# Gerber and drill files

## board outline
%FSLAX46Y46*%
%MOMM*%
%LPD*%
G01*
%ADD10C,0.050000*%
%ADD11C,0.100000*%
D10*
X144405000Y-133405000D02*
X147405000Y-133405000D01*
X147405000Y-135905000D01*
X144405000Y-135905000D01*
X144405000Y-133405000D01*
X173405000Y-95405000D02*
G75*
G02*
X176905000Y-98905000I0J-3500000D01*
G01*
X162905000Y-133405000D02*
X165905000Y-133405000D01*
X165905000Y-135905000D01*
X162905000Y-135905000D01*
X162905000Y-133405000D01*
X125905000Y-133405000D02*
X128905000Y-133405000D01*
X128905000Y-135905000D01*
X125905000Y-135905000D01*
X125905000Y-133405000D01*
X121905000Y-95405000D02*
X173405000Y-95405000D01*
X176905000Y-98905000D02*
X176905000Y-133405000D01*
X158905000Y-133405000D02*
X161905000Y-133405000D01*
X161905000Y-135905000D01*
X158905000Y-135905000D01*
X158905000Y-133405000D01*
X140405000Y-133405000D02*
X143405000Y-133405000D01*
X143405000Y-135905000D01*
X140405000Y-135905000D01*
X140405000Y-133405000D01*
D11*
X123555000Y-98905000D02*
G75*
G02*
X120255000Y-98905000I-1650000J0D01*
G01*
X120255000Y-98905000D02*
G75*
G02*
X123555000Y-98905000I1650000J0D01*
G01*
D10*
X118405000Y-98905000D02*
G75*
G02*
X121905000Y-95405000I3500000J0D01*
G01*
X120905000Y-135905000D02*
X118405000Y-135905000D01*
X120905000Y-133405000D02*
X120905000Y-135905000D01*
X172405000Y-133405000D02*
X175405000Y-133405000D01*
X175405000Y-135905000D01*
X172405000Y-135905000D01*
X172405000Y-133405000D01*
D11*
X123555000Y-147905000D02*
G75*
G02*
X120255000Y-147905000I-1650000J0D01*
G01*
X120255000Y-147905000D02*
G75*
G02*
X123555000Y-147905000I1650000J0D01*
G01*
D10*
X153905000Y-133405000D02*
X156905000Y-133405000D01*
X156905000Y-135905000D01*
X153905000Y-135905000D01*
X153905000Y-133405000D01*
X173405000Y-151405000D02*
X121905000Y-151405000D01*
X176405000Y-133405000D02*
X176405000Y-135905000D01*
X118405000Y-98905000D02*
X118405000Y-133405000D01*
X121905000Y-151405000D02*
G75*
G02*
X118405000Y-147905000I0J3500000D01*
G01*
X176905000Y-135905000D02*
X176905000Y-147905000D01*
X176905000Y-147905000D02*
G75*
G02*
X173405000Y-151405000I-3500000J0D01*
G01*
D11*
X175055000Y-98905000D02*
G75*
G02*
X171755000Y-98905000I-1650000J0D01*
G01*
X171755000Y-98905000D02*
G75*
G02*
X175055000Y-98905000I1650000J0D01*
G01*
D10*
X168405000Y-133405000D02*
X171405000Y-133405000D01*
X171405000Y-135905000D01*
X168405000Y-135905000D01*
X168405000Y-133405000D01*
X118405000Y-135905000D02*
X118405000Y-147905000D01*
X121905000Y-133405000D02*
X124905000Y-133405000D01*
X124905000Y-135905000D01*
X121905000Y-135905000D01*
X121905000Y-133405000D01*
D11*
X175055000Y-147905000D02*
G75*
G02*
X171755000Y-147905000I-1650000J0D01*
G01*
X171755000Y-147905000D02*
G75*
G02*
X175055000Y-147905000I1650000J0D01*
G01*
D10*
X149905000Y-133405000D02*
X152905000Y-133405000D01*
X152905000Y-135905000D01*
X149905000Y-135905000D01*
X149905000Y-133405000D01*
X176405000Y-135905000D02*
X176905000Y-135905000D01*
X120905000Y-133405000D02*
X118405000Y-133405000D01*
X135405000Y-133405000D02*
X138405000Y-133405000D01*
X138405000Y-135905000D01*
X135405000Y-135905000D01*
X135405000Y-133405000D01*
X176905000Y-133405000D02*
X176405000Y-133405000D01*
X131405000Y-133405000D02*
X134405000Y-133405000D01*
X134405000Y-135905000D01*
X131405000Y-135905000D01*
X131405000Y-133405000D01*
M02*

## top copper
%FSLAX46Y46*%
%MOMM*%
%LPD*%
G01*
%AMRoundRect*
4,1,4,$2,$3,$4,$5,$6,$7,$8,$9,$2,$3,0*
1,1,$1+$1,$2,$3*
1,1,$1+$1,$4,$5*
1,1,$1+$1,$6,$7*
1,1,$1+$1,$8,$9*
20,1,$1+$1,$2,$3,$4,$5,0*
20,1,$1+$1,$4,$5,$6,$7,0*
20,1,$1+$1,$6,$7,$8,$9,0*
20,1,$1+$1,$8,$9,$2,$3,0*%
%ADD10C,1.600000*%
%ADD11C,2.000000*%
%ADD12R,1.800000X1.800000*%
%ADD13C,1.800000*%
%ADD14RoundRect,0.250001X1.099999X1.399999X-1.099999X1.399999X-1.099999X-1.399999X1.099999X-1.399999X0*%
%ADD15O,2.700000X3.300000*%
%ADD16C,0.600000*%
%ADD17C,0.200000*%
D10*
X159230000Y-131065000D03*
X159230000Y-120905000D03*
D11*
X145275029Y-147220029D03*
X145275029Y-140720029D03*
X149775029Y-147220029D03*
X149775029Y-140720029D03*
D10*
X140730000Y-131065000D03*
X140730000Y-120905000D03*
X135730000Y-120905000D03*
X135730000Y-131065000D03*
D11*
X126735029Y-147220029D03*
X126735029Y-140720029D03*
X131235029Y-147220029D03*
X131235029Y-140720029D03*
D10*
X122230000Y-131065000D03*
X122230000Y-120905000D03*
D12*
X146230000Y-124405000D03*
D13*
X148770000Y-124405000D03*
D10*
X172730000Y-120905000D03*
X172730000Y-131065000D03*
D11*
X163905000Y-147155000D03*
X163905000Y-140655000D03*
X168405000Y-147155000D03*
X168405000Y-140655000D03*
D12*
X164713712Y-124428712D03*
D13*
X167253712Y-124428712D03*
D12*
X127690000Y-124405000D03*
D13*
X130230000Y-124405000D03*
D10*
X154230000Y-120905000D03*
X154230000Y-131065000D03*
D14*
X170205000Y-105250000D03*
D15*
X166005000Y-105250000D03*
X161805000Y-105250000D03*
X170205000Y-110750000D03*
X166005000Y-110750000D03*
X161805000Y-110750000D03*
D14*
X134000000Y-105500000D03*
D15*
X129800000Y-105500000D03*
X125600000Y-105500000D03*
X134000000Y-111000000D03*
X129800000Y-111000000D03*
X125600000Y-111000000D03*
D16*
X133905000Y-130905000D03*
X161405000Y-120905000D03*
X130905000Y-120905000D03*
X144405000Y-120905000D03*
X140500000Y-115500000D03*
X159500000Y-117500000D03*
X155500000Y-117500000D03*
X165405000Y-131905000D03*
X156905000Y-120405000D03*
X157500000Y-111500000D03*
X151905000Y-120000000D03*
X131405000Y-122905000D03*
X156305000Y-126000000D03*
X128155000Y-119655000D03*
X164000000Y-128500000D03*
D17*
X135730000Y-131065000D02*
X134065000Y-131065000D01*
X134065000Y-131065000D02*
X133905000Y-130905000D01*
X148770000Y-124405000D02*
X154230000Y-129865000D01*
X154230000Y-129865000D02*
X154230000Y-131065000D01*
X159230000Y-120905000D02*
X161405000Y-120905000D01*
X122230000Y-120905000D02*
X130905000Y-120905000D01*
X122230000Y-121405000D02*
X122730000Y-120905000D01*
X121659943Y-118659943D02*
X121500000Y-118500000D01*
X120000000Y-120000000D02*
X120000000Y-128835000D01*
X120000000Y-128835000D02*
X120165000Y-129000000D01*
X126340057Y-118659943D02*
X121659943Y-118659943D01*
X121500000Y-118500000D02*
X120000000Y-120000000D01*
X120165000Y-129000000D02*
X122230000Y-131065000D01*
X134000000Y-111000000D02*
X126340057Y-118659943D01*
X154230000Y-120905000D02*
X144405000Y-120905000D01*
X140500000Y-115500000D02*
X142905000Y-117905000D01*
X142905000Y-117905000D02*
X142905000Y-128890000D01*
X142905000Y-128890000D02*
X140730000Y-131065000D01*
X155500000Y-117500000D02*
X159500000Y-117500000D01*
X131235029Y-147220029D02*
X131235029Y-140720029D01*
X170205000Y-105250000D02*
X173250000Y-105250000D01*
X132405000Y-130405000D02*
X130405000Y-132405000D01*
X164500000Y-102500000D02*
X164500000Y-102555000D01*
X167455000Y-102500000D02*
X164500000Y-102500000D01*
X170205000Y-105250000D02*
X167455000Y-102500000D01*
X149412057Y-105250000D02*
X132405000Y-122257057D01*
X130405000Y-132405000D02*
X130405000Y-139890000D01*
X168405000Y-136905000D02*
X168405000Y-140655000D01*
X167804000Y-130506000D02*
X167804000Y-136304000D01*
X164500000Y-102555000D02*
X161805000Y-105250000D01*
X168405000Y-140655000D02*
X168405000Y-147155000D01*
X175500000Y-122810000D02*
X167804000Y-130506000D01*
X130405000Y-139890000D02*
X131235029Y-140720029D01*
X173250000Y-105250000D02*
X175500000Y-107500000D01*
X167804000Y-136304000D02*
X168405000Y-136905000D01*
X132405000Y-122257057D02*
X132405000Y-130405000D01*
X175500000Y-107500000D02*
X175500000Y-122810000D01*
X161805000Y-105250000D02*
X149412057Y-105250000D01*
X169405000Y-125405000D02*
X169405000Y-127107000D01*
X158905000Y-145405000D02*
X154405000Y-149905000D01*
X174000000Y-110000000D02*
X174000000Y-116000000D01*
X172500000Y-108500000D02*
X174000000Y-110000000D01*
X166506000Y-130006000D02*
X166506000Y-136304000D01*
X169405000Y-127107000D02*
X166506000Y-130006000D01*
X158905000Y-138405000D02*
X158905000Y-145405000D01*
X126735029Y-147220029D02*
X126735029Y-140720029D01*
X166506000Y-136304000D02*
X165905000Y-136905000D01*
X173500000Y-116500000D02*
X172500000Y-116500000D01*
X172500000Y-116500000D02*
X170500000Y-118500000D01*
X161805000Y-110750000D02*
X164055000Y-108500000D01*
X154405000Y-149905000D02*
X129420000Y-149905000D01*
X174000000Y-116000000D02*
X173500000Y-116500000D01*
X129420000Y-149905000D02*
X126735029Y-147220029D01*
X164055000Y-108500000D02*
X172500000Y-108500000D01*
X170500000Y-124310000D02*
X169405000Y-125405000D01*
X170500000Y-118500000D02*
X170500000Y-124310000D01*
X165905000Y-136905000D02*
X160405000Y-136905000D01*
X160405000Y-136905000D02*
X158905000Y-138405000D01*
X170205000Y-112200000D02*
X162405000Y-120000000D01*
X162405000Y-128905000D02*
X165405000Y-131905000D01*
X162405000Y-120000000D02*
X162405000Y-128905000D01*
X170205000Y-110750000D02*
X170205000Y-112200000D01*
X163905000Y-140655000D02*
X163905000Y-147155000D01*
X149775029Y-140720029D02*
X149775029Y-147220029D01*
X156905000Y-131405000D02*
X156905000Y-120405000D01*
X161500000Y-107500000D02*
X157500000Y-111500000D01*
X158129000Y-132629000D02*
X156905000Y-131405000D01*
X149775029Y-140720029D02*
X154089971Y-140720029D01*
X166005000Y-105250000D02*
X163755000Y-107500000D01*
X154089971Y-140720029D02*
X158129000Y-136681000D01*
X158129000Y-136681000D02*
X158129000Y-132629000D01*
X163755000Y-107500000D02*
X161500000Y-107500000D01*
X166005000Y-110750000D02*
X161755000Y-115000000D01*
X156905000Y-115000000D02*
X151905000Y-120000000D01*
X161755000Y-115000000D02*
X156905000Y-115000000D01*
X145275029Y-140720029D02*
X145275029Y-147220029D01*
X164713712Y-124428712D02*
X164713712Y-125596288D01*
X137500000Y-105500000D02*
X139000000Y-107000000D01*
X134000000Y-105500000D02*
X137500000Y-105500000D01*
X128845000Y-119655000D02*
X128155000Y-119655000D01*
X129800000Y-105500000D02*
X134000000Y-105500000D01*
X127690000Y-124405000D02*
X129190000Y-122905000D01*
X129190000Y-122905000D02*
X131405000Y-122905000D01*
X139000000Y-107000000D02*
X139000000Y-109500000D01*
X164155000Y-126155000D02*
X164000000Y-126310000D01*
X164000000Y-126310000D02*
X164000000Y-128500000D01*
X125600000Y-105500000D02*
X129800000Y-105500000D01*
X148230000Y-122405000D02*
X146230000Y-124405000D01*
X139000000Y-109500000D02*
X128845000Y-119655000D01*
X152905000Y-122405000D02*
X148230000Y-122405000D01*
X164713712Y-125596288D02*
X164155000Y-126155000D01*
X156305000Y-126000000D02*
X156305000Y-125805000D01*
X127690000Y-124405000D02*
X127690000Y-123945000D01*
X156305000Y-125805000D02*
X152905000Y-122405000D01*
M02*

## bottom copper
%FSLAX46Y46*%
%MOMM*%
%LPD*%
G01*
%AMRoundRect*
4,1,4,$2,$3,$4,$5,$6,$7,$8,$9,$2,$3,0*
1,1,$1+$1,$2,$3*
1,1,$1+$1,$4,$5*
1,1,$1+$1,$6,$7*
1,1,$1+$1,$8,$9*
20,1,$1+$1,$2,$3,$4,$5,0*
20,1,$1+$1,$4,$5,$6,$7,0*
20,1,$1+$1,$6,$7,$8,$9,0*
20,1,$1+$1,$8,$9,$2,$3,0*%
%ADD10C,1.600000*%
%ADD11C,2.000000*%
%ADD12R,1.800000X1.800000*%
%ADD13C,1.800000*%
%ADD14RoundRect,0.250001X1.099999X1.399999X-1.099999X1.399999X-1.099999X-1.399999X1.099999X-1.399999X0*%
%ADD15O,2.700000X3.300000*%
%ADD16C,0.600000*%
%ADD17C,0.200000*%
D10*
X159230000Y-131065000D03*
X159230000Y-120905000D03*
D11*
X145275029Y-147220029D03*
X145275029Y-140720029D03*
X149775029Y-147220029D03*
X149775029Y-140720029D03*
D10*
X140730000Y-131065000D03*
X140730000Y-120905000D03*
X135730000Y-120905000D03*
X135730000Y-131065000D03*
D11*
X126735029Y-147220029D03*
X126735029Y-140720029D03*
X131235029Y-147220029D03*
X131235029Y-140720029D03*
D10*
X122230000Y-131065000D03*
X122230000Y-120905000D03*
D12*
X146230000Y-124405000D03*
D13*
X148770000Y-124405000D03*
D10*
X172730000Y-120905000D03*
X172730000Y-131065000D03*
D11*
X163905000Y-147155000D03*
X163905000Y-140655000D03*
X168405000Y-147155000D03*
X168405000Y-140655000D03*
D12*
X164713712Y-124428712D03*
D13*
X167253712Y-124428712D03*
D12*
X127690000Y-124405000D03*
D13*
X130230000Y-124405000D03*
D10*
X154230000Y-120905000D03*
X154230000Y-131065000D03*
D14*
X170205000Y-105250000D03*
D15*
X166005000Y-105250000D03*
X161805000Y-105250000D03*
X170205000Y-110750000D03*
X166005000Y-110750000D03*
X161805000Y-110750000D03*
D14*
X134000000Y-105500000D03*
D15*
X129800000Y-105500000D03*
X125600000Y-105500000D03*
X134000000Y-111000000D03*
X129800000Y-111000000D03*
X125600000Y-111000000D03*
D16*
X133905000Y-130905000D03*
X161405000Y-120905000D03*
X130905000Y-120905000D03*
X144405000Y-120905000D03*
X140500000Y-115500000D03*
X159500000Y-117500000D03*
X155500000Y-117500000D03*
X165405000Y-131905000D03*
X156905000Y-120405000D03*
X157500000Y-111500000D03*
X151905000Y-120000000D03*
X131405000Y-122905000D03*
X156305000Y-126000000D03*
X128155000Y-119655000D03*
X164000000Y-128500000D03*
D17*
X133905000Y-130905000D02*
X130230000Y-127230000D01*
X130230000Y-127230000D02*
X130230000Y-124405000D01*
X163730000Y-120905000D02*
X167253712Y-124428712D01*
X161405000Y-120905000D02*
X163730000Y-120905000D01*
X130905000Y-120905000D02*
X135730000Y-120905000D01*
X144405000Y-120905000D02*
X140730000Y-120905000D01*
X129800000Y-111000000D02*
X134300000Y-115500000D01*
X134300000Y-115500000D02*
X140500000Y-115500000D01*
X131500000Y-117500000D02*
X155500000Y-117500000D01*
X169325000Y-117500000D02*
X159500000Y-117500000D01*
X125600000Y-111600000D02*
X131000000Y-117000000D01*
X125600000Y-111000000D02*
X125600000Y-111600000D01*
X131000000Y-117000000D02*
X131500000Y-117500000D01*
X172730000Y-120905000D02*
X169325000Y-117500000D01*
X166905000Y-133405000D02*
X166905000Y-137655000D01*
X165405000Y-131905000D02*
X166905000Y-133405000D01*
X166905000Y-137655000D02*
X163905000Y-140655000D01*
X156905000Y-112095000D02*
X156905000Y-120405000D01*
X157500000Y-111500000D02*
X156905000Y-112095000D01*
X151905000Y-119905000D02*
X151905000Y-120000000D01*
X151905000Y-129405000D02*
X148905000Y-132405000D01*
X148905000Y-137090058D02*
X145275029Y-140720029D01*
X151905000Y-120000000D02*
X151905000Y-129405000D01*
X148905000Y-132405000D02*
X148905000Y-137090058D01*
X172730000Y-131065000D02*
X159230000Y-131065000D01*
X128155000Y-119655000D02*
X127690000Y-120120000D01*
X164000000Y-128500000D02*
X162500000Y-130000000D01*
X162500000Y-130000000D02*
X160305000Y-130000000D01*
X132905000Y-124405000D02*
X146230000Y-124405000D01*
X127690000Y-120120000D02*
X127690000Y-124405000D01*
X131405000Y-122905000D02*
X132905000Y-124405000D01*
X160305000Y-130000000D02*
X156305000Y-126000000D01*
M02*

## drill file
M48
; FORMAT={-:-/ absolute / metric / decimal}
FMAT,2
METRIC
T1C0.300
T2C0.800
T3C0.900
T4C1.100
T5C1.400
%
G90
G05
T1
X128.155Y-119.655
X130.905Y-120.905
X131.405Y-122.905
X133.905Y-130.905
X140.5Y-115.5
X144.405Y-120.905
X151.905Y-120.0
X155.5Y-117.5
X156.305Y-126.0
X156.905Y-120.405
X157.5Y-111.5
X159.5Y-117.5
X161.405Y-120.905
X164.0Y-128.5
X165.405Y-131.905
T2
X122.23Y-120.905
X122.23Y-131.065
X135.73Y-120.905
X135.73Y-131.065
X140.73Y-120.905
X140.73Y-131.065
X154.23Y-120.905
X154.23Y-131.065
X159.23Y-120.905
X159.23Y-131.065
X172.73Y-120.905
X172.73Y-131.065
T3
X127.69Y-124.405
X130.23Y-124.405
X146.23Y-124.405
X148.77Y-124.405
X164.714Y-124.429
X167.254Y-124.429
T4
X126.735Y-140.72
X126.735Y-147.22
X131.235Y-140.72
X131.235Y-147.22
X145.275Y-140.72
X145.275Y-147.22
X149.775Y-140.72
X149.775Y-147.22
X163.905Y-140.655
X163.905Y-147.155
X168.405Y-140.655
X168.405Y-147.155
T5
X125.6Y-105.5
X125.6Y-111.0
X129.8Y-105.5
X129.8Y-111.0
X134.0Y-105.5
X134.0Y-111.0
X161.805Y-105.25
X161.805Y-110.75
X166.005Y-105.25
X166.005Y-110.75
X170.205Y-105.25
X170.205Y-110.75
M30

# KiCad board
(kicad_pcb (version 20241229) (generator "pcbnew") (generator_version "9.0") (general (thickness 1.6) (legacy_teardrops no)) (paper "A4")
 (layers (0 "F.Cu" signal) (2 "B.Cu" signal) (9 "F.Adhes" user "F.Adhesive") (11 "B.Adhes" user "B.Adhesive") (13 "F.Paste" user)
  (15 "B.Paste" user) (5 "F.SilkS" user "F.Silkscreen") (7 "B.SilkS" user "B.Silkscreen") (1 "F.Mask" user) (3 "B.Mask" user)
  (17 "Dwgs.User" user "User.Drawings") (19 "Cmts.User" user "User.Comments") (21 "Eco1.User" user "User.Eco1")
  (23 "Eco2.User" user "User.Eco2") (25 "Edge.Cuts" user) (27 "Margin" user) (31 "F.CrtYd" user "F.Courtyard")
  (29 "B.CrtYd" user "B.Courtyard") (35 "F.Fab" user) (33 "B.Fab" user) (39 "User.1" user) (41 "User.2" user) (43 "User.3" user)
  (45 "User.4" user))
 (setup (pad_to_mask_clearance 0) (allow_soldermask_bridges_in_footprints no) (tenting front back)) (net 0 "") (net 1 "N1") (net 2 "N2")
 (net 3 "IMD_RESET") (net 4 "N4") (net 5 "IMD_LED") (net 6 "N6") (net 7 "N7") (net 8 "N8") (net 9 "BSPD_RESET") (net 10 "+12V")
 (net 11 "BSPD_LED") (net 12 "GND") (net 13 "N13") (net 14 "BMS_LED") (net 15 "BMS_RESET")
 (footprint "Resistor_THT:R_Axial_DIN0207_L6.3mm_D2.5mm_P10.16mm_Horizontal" (layer "F.Cu") (at 159.23 131.065 90)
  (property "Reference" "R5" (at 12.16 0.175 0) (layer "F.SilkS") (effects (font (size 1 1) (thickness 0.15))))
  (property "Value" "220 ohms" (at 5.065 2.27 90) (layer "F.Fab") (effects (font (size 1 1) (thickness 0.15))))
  (pad "1" thru_hole circle (at 0 0 90) (size 1.6 1.6) (drill 0.8) (layers "*.Cu" "*.Mask") (remove_unused_layers no) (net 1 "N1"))
  (pad "2" thru_hole circle (at 10.16 0 90) (size 1.6 1.6) (drill 0.8) (layers "*.Cu" "*.Mask") (remove_unused_layers no) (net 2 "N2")))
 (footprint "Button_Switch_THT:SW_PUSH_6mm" (layer "F.Cu") (at 145.275029 147.220029 90)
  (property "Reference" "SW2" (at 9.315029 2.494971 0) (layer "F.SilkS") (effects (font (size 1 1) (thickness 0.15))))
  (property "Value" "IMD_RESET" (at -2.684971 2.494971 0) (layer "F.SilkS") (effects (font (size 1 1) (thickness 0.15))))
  (pad "1" thru_hole circle (at 0 0 180) (size 2 2) (drill 1.1) (layers "*.Cu" "*.Mask") (remove_unused_layers no) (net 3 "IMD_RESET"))
  (pad "1" thru_hole circle (at 6.5 0 180) (size 2 2) (drill 1.1) (layers "*.Cu" "*.Mask") (remove_unused_layers no) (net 3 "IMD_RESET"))
  (pad "2" thru_hole circle (at 0 4.5 180) (size 2 2) (drill 1.1) (layers "*.Cu" "*.Mask") (remove_unused_layers no) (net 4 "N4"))
  (pad "2" thru_hole circle (at 6.5 4.5 180) (size 2 2) (drill 1.1) (layers "*.Cu" "*.Mask") (remove_unused_layers no) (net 4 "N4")))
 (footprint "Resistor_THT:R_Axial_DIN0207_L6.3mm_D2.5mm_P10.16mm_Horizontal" (layer "F.Cu") (at 140.73 131.065 90)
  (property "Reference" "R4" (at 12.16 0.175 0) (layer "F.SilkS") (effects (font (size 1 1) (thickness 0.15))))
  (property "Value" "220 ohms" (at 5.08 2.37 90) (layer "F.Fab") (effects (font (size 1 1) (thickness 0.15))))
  (pad "1" thru_hole circle (at 0 0 90) (size 1.6 1.6) (drill 0.8) (layers "*.Cu" "*.Mask") (remove_unused_layers no) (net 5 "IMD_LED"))
  (pad "2" thru_hole circle (at 10.16 0 90) (size 1.6 1.6) (drill 0.8) (layers "*.Cu" "*.Mask") (remove_unused_layers no) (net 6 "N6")))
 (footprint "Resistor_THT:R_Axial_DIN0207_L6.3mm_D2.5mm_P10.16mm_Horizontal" (layer "F.Cu") (at 135.73 120.905 -90)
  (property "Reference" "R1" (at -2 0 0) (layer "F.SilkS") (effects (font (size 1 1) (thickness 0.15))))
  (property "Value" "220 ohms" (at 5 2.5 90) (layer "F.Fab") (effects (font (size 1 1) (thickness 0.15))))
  (pad "1" thru_hole circle (at 0 0 270) (size 1.6 1.6) (drill 0.8) (layers "*.Cu" "*.Mask") (remove_unused_layers no) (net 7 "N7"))
  (pad "2" thru_hole circle (at 10.16 0 270) (size 1.6 1.6) (drill 0.8) (layers "*.Cu" "*.Mask") (remove_unused_layers no) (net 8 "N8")))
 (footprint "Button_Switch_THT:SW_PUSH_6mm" (layer "F.Cu") (at 126.735029 147.220029 90)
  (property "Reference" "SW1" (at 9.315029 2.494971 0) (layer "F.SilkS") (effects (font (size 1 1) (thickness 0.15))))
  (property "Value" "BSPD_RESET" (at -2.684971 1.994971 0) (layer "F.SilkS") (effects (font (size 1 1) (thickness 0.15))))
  (pad "1" thru_hole circle (at 0 0 180) (size 2 2) (drill 1.1) (layers "*.Cu" "*.Mask") (remove_unused_layers no) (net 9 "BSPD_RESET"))
  (pad "1" thru_hole circle (at 6.5 0 180) (size 2 2) (drill 1.1) (layers "*.Cu" "*.Mask") (remove_unused_layers no) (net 9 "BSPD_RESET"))
  (pad "2" thru_hole circle (at 0 4.5 180) (size 2 2) (drill 1.1) (layers "*.Cu" "*.Mask") (remove_unused_layers no) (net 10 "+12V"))
  (pad "2" thru_hole circle (at 6.5 4.5 180) (size 2 2) (drill 1.1) (layers "*.Cu" "*.Mask") (remove_unused_layers no) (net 10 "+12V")))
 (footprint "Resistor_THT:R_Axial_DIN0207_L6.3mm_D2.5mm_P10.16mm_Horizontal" (layer "F.Cu") (at 122.23 131.065 90)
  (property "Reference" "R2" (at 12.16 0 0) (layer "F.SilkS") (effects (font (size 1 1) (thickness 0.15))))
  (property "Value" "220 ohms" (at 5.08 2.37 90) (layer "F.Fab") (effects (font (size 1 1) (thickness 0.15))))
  (pad "1" thru_hole circle (at 0 0 90) (size 1.6 1.6) (drill 0.8) (layers "*.Cu" "*.Mask") (remove_unused_layers no) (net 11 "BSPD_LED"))
  (pad "2" thru_hole circle (at 10.16 0 90) (size 1.6 1.6) (drill 0.8) (layers "*.Cu" "*.Mask") (remove_unused_layers no) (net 7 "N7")))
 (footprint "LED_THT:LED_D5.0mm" (layer "F.Cu") (at 146.23 124.405)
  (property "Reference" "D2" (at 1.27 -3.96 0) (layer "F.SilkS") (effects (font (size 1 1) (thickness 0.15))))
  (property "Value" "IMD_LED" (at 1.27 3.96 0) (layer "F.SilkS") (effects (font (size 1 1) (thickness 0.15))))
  (pad "1" thru_hole rect (at 0 0) (size 1.8 1.8) (drill 0.9) (layers "*.Cu" "*.Mask") (remove_unused_layers no) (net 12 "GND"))
  (pad "2" thru_hole circle (at 2.54 0) (size 1.8 1.8) (drill 0.9) (layers "*.Cu" "*.Mask") (remove_unused_layers no) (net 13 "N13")))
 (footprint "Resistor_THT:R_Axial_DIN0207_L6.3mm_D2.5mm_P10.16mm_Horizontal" (layer "F.Cu") (at 172.73 120.905 -90)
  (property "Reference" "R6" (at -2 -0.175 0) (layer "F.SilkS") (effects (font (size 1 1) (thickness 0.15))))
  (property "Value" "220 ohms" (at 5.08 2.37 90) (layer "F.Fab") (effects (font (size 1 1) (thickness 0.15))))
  (pad "1" thru_hole circle (at 0 0 270) (size 1.6 1.6) (drill 0.8) (layers "*.Cu" "*.Mask") (remove_unused_layers no) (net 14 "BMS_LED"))
  (pad "2" thru_hole circle (at 10.16 0 270) (size 1.6 1.6) (drill 0.8) (layers "*.Cu" "*.Mask") (remove_unused_layers no) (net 1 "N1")))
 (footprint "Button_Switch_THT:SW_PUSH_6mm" (layer "F.Cu") (at 163.905 147.155 90)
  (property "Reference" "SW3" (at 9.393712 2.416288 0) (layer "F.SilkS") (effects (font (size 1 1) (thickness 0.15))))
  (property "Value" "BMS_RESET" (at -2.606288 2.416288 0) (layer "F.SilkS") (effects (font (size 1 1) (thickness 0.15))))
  (pad "1" thru_hole circle (at 0 0 180) (size 2 2) (drill 1.1) (layers "*.Cu" "*.Mask") (remove_unused_layers no) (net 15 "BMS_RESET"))
  (pad "1" thru_hole circle (at 6.5 0 180) (size 2 2) (drill 1.1) (layers "*.Cu" "*.Mask") (remove_unused_layers no) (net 15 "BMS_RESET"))
  (pad "2" thru_hole circle (at 0 4.5 180) (size 2 2) (drill 1.1) (layers "*.Cu" "*.Mask") (remove_unused_layers no) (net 10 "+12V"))
  (pad "2" thru_hole circle (at 6.5 4.5 180) (size 2 2) (drill 1.1) (layers "*.Cu" "*.Mask") (remove_unused_layers no) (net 10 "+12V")))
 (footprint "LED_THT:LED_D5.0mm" (layer "F.Cu") (at 164.713712 124.428712)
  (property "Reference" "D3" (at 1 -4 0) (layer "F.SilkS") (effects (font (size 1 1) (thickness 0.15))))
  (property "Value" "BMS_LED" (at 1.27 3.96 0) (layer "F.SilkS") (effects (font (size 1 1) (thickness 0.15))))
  (pad "1" thru_hole rect (at 0 0) (size 1.8 1.8) (drill 0.9) (layers "*.Cu" "*.Mask") (remove_unused_layers no) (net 12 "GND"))
  (pad "2" thru_hole circle (at 2.54 0) (size 1.8 1.8) (drill 0.9) (layers "*.Cu" "*.Mask") (remove_unused_layers no) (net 2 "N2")))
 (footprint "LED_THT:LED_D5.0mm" (layer "F.Cu") (at 127.69 124.405)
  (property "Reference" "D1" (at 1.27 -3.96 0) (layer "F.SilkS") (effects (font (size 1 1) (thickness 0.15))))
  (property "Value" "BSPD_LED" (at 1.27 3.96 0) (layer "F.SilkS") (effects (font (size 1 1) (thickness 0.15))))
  (pad "1" thru_hole rect (at 0 0) (size 1.8 1.8) (drill 0.9) (layers "*.Cu" "*.Mask") (remove_unused_layers no) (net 12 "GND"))
  (pad "2" thru_hole circle (at 2.54 0) (size 1.8 1.8) (drill 0.9) (layers "*.Cu" "*.Mask") (remove_unused_layers no) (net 8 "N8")))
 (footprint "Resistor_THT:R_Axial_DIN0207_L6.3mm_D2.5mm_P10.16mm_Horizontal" (layer "F.Cu") (at 154.23 120.905 -90)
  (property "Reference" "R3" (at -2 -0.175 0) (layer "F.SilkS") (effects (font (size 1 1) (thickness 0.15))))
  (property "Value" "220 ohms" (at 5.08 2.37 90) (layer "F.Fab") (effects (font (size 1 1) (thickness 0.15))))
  (pad "1" thru_hole circle (at 0 0 270) (size 1.6 1.6) (drill 0.8) (layers "*.Cu" "*.Mask") (remove_unused_layers no) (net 6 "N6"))
  (pad "2" thru_hole circle (at 10.16 0 270) (size 1.6 1.6) (drill 0.8) (layers "*.Cu" "*.Mask") (remove_unused_layers no) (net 13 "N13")))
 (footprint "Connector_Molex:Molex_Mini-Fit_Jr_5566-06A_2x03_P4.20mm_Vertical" (layer "B.Cu") (at 170.205 105.25 180)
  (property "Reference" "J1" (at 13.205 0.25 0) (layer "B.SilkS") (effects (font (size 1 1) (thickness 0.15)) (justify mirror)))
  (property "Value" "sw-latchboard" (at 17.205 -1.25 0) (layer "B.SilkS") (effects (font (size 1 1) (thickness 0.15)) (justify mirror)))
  (pad "1" thru_hole roundrect (at 0 0 180) (size 2.7 3.3) (drill 1.4) (layers "*.Cu" "*.Mask") (remove_unused_layers no)
   (roundrect_rratio 0.092593) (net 10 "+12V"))
  (pad "2" thru_hole oval (at 4.2 0 180) (size 2.7 3.3) (drill 1.4) (layers "*.Cu" "*.Mask") (remove_unused_layers no) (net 4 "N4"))
  (pad "3" thru_hole oval (at 8.4 0 180) (size 2.7 3.3) (drill 1.4) (layers "*.Cu" "*.Mask") (remove_unused_layers no) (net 10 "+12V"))
  (pad "4" thru_hole oval (at 0 -5.5 180) (size 2.7 3.3) (drill 1.4) (layers "*.Cu" "*.Mask") (remove_unused_layers no) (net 15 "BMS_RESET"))
  (pad "5" thru_hole oval (at 4.2 -5.5 180) (size 2.7 3.3) (drill 1.4) (layers "*.Cu" "*.Mask") (remove_unused_layers no)
   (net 3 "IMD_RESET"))
  (pad "6" thru_hole oval (at 8.4 -5.5 180) (size 2.7 3.3) (drill 1.4) (layers "*.Cu" "*.Mask") (remove_unused_layers no)
   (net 9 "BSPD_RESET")))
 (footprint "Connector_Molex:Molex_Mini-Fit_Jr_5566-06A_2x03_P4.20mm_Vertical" (layer "B.Cu") (at 134 105.5 180)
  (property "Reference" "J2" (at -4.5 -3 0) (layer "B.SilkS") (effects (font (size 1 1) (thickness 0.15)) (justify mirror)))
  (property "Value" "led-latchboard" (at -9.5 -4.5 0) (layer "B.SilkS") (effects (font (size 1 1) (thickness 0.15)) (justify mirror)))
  (pad "1" thru_hole roundrect (at 0 0 180) (size 2.7 3.3) (drill 1.4) (layers "*.Cu" "*.Mask") (remove_unused_layers no)
   (roundrect_rratio 0.092593) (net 12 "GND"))
  (pad "2" thru_hole oval (at 4.2 0 180) (size 2.7 3.3) (drill 1.4) (layers "*.Cu" "*.Mask") (remove_unused_layers no) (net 12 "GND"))
  (pad "3" thru_hole oval (at 8.4 0 180) (size 2.7 3.3) (drill 1.4) (layers "*.Cu" "*.Mask") (remove_unused_layers no) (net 12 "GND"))
  (pad "4" thru_hole oval (at 0 -5.5 180) (size 2.7 3.3) (drill 1.4) (layers "*.Cu" "*.Mask") (remove_unused_layers no) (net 11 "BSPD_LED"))
  (pad "5" thru_hole oval (at 4.2 -5.5 180) (size 2.7 3.3) (drill 1.4) (layers "*.Cu" "*.Mask") (remove_unused_layers no) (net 5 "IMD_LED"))
  (pad "6" thru_hole oval (at 8.4 -5.5 180) (size 2.7 3.3) (drill 1.4) (layers "*.Cu" "*.Mask") (remove_unused_layers no) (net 14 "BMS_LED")))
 (gr_rect (start 144.405 133.405) (end 147.405 135.905) (stroke (width 0.05) (type default)) (fill no) (layer "Edge.Cuts"))
 (gr_arc (start 173.405 95.405) (mid 175.879874 96.430126) (end 176.905 98.905) (stroke (width 0.05) (type default)) (layer "Edge.Cuts"))
 (gr_rect (start 162.905 133.405) (end 165.905 135.905) (stroke (width 0.05) (type default)) (fill no) (layer "Edge.Cuts"))
 (gr_rect (start 125.905 133.405) (end 128.905 135.905) (stroke (width 0.05) (type default)) (fill no) (layer "Edge.Cuts"))
 (gr_line (start 121.905 95.405) (end 173.405 95.405) (stroke (width 0.05) (type default)) (layer "Edge.Cuts"))
 (gr_line (start 176.905 98.905) (end 176.905 133.405) (stroke (width 0.05) (type default)) (layer "Edge.Cuts"))
 (gr_rect (start 158.905 133.405) (end 161.905 135.905) (stroke (width 0.05) (type default)) (fill no) (layer "Edge.Cuts"))
 (gr_rect (start 140.405 133.405) (end 143.405 135.905) (stroke (width 0.05) (type default)) (fill no) (layer "Edge.Cuts"))
 (gr_circle (center 121.905 98.905) (end 123.555 98.905) (stroke (width 0.1) (type solid)) (fill no) (layer "Edge.Cuts"))
 (gr_arc (start 118.405 98.905) (mid 119.430126 96.430126) (end 121.905 95.405) (stroke (width 0.05) (type default)) (layer "Edge.Cuts"))
 (gr_line (start 120.905 135.905) (end 118.405 135.905) (stroke (width 0.05) (type default)) (layer "Edge.Cuts"))
 (gr_line (start 120.905 133.405) (end 120.905 135.905) (stroke (width 0.05) (type default)) (layer "Edge.Cuts"))
 (gr_rect (start 172.405 133.405) (end 175.405 135.905) (stroke (width 0.05) (type default)) (fill no) (layer "Edge.Cuts"))
 (gr_circle (center 121.905 147.905) (end 123.555 147.905) (stroke (width 0.1) (type solid)) (fill no) (layer "Edge.Cuts"))
 (gr_rect (start 153.905 133.405) (end 156.905 135.905) (stroke (width 0.05) (type default)) (fill no) (layer "Edge.Cuts"))
 (gr_line (start 173.405 151.405) (end 121.905 151.405) (stroke (width 0.05) (type default)) (layer "Edge.Cuts"))
 (gr_line (start 176.405 133.405) (end 176.405 135.905) (stroke (width 0.05) (type default)) (layer "Edge.Cuts"))
 (gr_line (start 118.405 98.905) (end 118.405 133.405) (stroke (width 0.05) (type default)) (layer "Edge.Cuts"))
 (gr_arc (start 121.905 151.405) (mid 119.430126 150.379874) (end 118.405 147.905) (stroke (width 0.05) (type default)) (layer "Edge.Cuts"))
 (gr_line (start 176.905 135.905) (end 176.905 147.905) (stroke (width 0.05) (type default)) (layer "Edge.Cuts"))
 (gr_arc (start 176.905 147.905) (mid 175.879874 150.379874) (end 173.405 151.405) (stroke (width 0.05) (type default)) (layer "Edge.Cuts"))
 (gr_circle (center 173.405 98.905) (end 175.055 98.905) (stroke (width 0.1) (type solid)) (fill no) (layer "Edge.Cuts"))
 (gr_rect (start 168.405 133.405) (end 171.405 135.905) (stroke (width 0.05) (type default)) (fill no) (layer "Edge.Cuts"))
 (gr_line (start 118.405 135.905) (end 118.405 147.905) (stroke (width 0.05) (type default)) (layer "Edge.Cuts"))
 (gr_rect (start 121.905 133.405) (end 124.905 135.905) (stroke (width 0.05) (type default)) (fill no) (layer "Edge.Cuts"))
 (gr_circle (center 173.405 147.905) (end 175.055 147.905) (stroke (width 0.1) (type solid)) (fill no) (layer "Edge.Cuts"))
 (gr_rect (start 149.905 133.405) (end 152.905 135.905) (stroke (width 0.05) (type default)) (fill no) (layer "Edge.Cuts"))
 (gr_line (start 176.405 135.905) (end 176.905 135.905) (stroke (width 0.05) (type default)) (layer "Edge.Cuts"))
 (gr_line (start 120.905 133.405) (end 118.405 133.405) (stroke (width 0.05) (type default)) (layer "Edge.Cuts"))
 (gr_rect (start 135.405 133.405) (end 138.405 135.905) (stroke (width 0.05) (type default)) (fill no) (layer "Edge.Cuts"))
 (gr_line (start 176.905 133.405) (end 176.405 133.405) (stroke (width 0.05) (type default)) (layer "Edge.Cuts"))
 (gr_rect (start 131.405 133.405) (end 134.405 135.905) (stroke (width 0.05) (type default)) (fill no) (layer "Edge.Cuts"))
 (segment (start 135.73 131.065) (end 134.065 131.065) (width 0.2) (layer "F.Cu") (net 8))
 (segment (start 134.065 131.065) (end 133.905 130.905) (width 0.2) (layer "F.Cu") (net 8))
 (via (at 133.905 130.905) (size 0.6) (drill 0.3) (layers "F.Cu" "B.Cu") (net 8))
 (segment (start 133.905 130.905) (end 130.23 127.23) (width 0.2) (layer "B.Cu") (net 8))
 (segment (start 130.23 127.23) (end 130.23 124.405) (width 0.2) (layer "B.Cu") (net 8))
 (segment (start 148.77 124.405) (end 154.23 129.865) (width 0.2) (layer "F.Cu") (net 13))
 (segment (start 154.23 129.865) (end 154.23 131.065) (width 0.2) (layer "F.Cu") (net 13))
 (segment (start 159.23 120.905) (end 161.405 120.905) (width 0.2) (layer "F.Cu") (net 2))
 (via (at 161.405 120.905) (size 0.6) (drill 0.3) (layers "F.Cu" "B.Cu") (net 2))
 (segment (start 163.73 120.905) (end 167.253712 124.428712) (width 0.2) (layer "B.Cu") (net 2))
 (segment (start 161.405 120.905) (end 163.73 120.905) (width 0.2) (layer "B.Cu") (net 2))
 (segment (start 122.23 120.905) (end 130.905 120.905) (width 0.2) (layer "F.Cu") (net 7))
 (segment (start 122.23 121.405) (end 122.73 120.905) (width 0.2) (layer "F.Cu") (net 7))
 (via (at 130.905 120.905) (size 0.6) (drill 0.3) (layers "F.Cu" "B.Cu") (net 7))
 (segment (start 130.905 120.905) (end 135.73 120.905) (width 0.2) (layer "B.Cu") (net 7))
 (segment (start 121.659943 118.659943) (end 121.5 118.5) (width 0.2) (layer "F.Cu") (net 11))
 (segment (start 120 120) (end 120 128.835) (width 0.2) (layer "F.Cu") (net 11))
 (segment (start 120 128.835) (end 120.165 129) (width 0.2) (layer "F.Cu") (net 11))
 (segment (start 126.340057 118.659943) (end 121.659943 118.659943) (width 0.2) (layer "F.Cu") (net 11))
 (segment (start 121.5 118.5) (end 120 120) (width 0.2) (layer "F.Cu") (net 11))
 (segment (start 120.165 129) (end 122.23 131.065) (width 0.2) (layer "F.Cu") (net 11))
 (segment (start 134 111) (end 126.340057 118.659943) (width 0.2) (layer "F.Cu") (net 11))
 (segment (start 154.23 120.905) (end 144.405 120.905) (width 0.2) (layer "F.Cu") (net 6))
 (via (at 144.405 120.905) (size 0.6) (drill 0.3) (layers "F.Cu" "B.Cu") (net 6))
 (segment (start 144.405 120.905) (end 140.73 120.905) (width 0.2) (layer "B.Cu") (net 6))
 (segment (start 140.5 115.5) (end 142.905 117.905) (width 0.2) (layer "F.Cu") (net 5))
 (segment (start 142.905 117.905) (end 142.905 128.89) (width 0.2) (layer "F.Cu") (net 5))
 (segment (start 142.905 128.89) (end 140.73 131.065) (width 0.2) (layer "F.Cu") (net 5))
 (via (at 140.5 115.5) (size 0.6) (drill 0.3) (layers "F.Cu" "B.Cu") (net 5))
 (segment (start 129.8 111) (end 134.3 115.5) (width 0.2) (layer "B.Cu") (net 5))
 (segment (start 134.3 115.5) (end 140.5 115.5) (width 0.2) (layer "B.Cu") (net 5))
 (segment (start 155.5 117.5) (end 159.5 117.5) (width 0.2) (layer "F.Cu") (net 14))
 (via (at 159.5 117.5) (size 0.6) (drill 0.3) (layers "F.Cu" "B.Cu") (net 14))
 (via (at 155.5 117.5) (size 0.6) (drill 0.3) (layers "F.Cu" "B.Cu") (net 14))
 (segment (start 131.5 117.5) (end 155.5 117.5) (width 0.2) (layer "B.Cu") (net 14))
 (segment (start 169.325 117.5) (end 159.5 117.5) (width 0.2) (layer "B.Cu") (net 14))
 (segment (start 125.6 111.6) (end 131 117) (width 0.2) (layer "B.Cu") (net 14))
 (segment (start 125.6 111) (end 125.6 111.6) (width 0.2) (layer "B.Cu") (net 14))
 (segment (start 131 117) (end 131.5 117.5) (width 0.2) (layer "B.Cu") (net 14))
 (segment (start 172.73 120.905) (end 169.325 117.5) (width 0.2) (layer "B.Cu") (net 14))
 (segment (start 131.235029 147.220029) (end 131.235029 140.720029) (width 0.2) (layer "F.Cu") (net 10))
 (segment (start 170.205 105.25) (end 173.25 105.25) (width 0.2) (layer "F.Cu") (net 10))
 (segment (start 132.405 130.405) (end 130.405 132.405) (width 0.2) (layer "F.Cu") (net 10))
 (segment (start 164.5 102.5) (end 164.5 102.555) (width 0.2) (layer "F.Cu") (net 10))
 (segment (start 167.455 102.5) (end 164.5 102.5) (width 0.2) (layer "F.Cu") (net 10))
 (segment (start 170.205 105.25) (end 167.455 102.5) (width 0.2) (layer "F.Cu") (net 10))
 (segment (start 149.412057 105.25) (end 132.405 122.257057) (width 0.2) (layer "F.Cu") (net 10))
 (segment (start 130.405 132.405) (end 130.405 139.89) (width 0.2) (layer "F.Cu") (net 10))
 (segment (start 168.405 136.905) (end 168.405 140.655) (width 0.2) (layer "F.Cu") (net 10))
 (segment (start 167.804 130.506) (end 167.804 136.304) (width 0.2) (layer "F.Cu") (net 10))
 (segment (start 164.5 102.555) (end 161.805 105.25) (width 0.2) (layer "F.Cu") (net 10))
 (segment (start 168.405 140.655) (end 168.405 147.155) (width 0.2) (layer "F.Cu") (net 10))
 (segment (start 175.5 122.81) (end 167.804 130.506) (width 0.2) (layer "F.Cu") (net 10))
 (segment (start 130.405 139.89) (end 131.235029 140.720029) (width 0.2) (layer "F.Cu") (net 10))
 (segment (start 173.25 105.25) (end 175.5 107.5) (width 0.2) (layer "F.Cu") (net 10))
 (segment (start 167.804 136.304) (end 168.405 136.905) (width 0.2) (layer "F.Cu") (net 10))
 (segment (start 132.405 122.257057) (end 132.405 130.405) (width 0.2) (layer "F.Cu") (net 10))
 (segment (start 175.5 107.5) (end 175.5 122.81) (width 0.2) (layer "F.Cu") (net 10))
 (segment (start 161.805 105.25) (end 149.412057 105.25) (width 0.2) (layer "F.Cu") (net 10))
 (segment (start 169.405 125.405) (end 169.405 127.107) (width 0.2) (layer "F.Cu") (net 9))
 (segment (start 158.905 145.405) (end 154.405 149.905) (width 0.2) (layer "F.Cu") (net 9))
 (segment (start 174 110) (end 174 116) (width 0.2) (layer "F.Cu") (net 9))
 (segment (start 172.5 108.5) (end 174 110) (width 0.2) (layer "F.Cu") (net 9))
 (segment (start 166.506 130.006) (end 166.506 136.304) (width 0.2) (layer "F.Cu") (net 9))
 (segment (start 169.405 127.107) (end 166.506 130.006) (width 0.2) (layer "F.Cu") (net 9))
 (segment (start 158.905 138.405) (end 158.905 145.405) (width 0.2) (layer "F.Cu") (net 9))
 (segment (start 126.735029 147.220029) (end 126.735029 140.720029) (width 0.2) (layer "F.Cu") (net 9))
 (segment (start 166.506 136.304) (end 165.905 136.905) (width 0.2) (layer "F.Cu") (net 9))
 (segment (start 173.5 116.5) (end 172.5 116.5) (width 0.2) (layer "F.Cu") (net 9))
 (segment (start 172.5 116.5) (end 170.5 118.5) (width 0.2) (layer "F.Cu") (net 9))
 (segment (start 161.805 110.75) (end 164.055 108.5) (width 0.2) (layer "F.Cu") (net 9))
 (segment (start 154.405 149.905) (end 129.42 149.905) (width 0.2) (layer "F.Cu") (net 9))
 (segment (start 174 116) (end 173.5 116.5) (width 0.2) (layer "F.Cu") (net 9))
 (segment (start 129.42 149.905) (end 126.735029 147.220029) (width 0.2) (layer "F.Cu") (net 9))
 (segment (start 164.055 108.5) (end 172.5 108.5) (width 0.2) (layer "F.Cu") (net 9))
 (segment (start 170.5 124.31) (end 169.405 125.405) (width 0.2) (layer "F.Cu") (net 9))
 (segment (start 170.5 118.5) (end 170.5 124.31) (width 0.2) (layer "F.Cu") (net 9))
 (segment (start 165.905 136.905) (end 160.405 136.905) (width 0.2) (layer "F.Cu") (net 9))
 (segment (start 160.405 136.905) (end 158.905 138.405) (width 0.2) (layer "F.Cu") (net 9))
 (segment (start 170.205 112.2) (end 162.405 120) (width 0.2) (layer "F.Cu") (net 15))
 (segment (start 162.405 128.905) (end 165.405 131.905) (width 0.2) (layer "F.Cu") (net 15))
 (segment (start 162.405 120) (end 162.405 128.905) (width 0.2) (layer "F.Cu") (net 15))
 (segment (start 170.205 110.75) (end 170.205 112.2) (width 0.2) (layer "F.Cu") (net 15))
 (segment (start 163.905 140.655) (end 163.905 147.155) (width 0.2) (layer "F.Cu") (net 15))
 (via (at 165.405 131.905) (size 0.6) (drill 0.3) (layers "F.Cu" "B.Cu") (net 15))
 (segment (start 166.905 133.405) (end 166.905 137.655) (width 0.2) (layer "B.Cu") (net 15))
 (segment (start 165.405 131.905) (end 166.905 133.405) (width 0.2) (layer "B.Cu") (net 15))
 (segment (start 166.905 137.655) (end 163.905 140.655) (width 0.2) (layer "B.Cu") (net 15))
 (segment (start 149.775029 140.720029) (end 149.775029 147.220029) (width 0.2) (layer "F.Cu") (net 4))
 (segment (start 156.905 131.405) (end 156.905 120.405) (width 0.2) (layer "F.Cu") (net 4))
 (segment (start 161.5 107.5) (end 157.5 111.5) (width 0.2) (layer "F.Cu") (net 4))
 (segment (start 158.129 132.629) (end 156.905 131.405) (width 0.2) (layer "F.Cu") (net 4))
 (segment (start 149.775029 140.720029) (end 154.089971 140.720029) (width 0.2) (layer "F.Cu") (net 4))
 (segment (start 166.005 105.25) (end 163.755 107.5) (width 0.2) (layer "F.Cu") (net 4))
 (segment (start 154.089971 140.720029) (end 158.129 136.681) (width 0.2) (layer "F.Cu") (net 4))
 (segment (start 158.129 136.681) (end 158.129 132.629) (width 0.2) (layer "F.Cu") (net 4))
 (segment (start 163.755 107.5) (end 161.5 107.5) (width 0.2) (layer "F.Cu") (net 4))
 (via (at 156.905 120.405) (size 0.6) (drill 0.3) (layers "F.Cu" "B.Cu") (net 4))
 (via (at 157.5 111.5) (size 0.6) (drill 0.3) (layers "F.Cu" "B.Cu") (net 4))
 (segment (start 156.905 112.095) (end 156.905 120.405) (width 0.2) (layer "B.Cu") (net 4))
 (segment (start 157.5 111.5) (end 156.905 112.095) (width 0.2) (layer "B.Cu") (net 4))
 (segment (start 166.005 110.75) (end 161.755 115) (width 0.2) (layer "F.Cu") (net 3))
 (segment (start 156.905 115) (end 151.905 120) (width 0.2) (layer "F.Cu") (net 3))
 (segment (start 161.755 115) (end 156.905 115) (width 0.2) (layer "F.Cu") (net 3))
 (segment (start 145.275029 140.720029) (end 145.275029 147.220029) (width 0.2) (layer "F.Cu") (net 3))
 (via (at 151.905 120) (size 0.6) (drill 0.3) (layers "F.Cu" "B.Cu") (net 3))
 (segment (start 151.905 119.905) (end 151.905 120) (width 0.2) (layer "B.Cu") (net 3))
 (segment (start 151.905 129.405) (end 148.905 132.405) (width 0.2) (layer "B.Cu") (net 3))
 (segment (start 148.905 137.090058) (end 145.275029 140.720029) (width 0.2) (layer "B.Cu") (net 3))
 (segment (start 151.905 120) (end 151.905 129.405) (width 0.2) (layer "B.Cu") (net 3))
 (segment (start 148.905 132.405) (end 148.905 137.090058) (width 0.2) (layer "B.Cu") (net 3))
 (segment (start 172.73 131.065) (end 159.23 131.065) (width 0.2) (layer "B.Cu") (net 1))
 (segment (start 164.713712 124.428712) (end 164.713712 125.596288) (width 0.2) (layer "F.Cu") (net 12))
 (segment (start 137.5 105.5) (end 139 107) (width 0.2) (layer "F.Cu") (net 12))
 (segment (start 134 105.5) (end 137.5 105.5) (width 0.2) (layer "F.Cu") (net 12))
 (segment (start 128.845 119.655) (end 128.155 119.655) (width 0.2) (layer "F.Cu") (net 12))
 (segment (start 129.8 105.5) (end 134 105.5) (width 0.2) (layer "F.Cu") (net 12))
 (segment (start 127.69 124.405) (end 129.19 122.905) (width 0.2) (layer "F.Cu") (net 12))
 (segment (start 129.19 122.905) (end 131.405 122.905) (width 0.2) (layer "F.Cu") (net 12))
 (segment (start 139 107) (end 139 109.5) (width 0.2) (layer "F.Cu") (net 12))
 (segment (start 164.155 126.155) (end 164 126.31) (width 0.2) (layer "F.Cu") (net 12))
 (segment (start 164 126.31) (end 164 128.5) (width 0.2) (layer "F.Cu") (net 12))
 (segment (start 125.6 105.5) (end 129.8 105.5) (width 0.2) (layer "F.Cu") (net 12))
 (segment (start 148.23 122.405) (end 146.23 124.405) (width 0.2) (layer "F.Cu") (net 12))
 (segment (start 139 109.5) (end 128.845 119.655) (width 0.2) (layer "F.Cu") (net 12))
 (segment (start 152.905 122.405) (end 148.23 122.405) (width 0.2) (layer "F.Cu") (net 12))
 (segment (start 164.713712 125.596288) (end 164.155 126.155) (width 0.2) (layer "F.Cu") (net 12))
 (segment (start 156.305 126) (end 156.305 125.805) (width 0.2) (layer "F.Cu") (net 12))
 (segment (start 127.69 124.405) (end 127.69 123.945) (width 0.2) (layer "F.Cu") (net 12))
 (segment (start 156.305 125.805) (end 152.905 122.405) (width 0.2) (layer "F.Cu") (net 12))
 (via (at 131.405 122.905) (size 0.6) (drill 0.3) (layers "F.Cu" "B.Cu") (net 12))
 (via (at 156.305 126) (size 0.6) (drill 0.3) (layers "F.Cu" "B.Cu") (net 12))
 (via (at 128.155 119.655) (size 0.6) (drill 0.3) (layers "F.Cu" "B.Cu") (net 12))
 (via (at 164 128.5) (size 0.6) (drill 0.3) (layers "F.Cu" "B.Cu") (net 12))
 (segment (start 128.155 119.655) (end 127.69 120.12) (width 0.2) (layer "B.Cu") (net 12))
 (segment (start 164 128.5) (end 162.5 130) (width 0.2) (layer "B.Cu") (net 12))
 (segment (start 162.5 130) (end 160.305 130) (width 0.2) (layer "B.Cu") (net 12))
 (segment (start 132.905 124.405) (end 146.23 124.405) (width 0.2) (layer "B.Cu") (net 12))
 (segment (start 127.69 120.12) (end 127.69 124.405) (width 0.2) (layer "B.Cu") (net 12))
 (segment (start 131.405 122.905) (end 132.905 124.405) (width 0.2) (layer "B.Cu") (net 12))
 (segment (start 160.305 130) (end 156.305 126) (width 0.2) (layer "B.Cu") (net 12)))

